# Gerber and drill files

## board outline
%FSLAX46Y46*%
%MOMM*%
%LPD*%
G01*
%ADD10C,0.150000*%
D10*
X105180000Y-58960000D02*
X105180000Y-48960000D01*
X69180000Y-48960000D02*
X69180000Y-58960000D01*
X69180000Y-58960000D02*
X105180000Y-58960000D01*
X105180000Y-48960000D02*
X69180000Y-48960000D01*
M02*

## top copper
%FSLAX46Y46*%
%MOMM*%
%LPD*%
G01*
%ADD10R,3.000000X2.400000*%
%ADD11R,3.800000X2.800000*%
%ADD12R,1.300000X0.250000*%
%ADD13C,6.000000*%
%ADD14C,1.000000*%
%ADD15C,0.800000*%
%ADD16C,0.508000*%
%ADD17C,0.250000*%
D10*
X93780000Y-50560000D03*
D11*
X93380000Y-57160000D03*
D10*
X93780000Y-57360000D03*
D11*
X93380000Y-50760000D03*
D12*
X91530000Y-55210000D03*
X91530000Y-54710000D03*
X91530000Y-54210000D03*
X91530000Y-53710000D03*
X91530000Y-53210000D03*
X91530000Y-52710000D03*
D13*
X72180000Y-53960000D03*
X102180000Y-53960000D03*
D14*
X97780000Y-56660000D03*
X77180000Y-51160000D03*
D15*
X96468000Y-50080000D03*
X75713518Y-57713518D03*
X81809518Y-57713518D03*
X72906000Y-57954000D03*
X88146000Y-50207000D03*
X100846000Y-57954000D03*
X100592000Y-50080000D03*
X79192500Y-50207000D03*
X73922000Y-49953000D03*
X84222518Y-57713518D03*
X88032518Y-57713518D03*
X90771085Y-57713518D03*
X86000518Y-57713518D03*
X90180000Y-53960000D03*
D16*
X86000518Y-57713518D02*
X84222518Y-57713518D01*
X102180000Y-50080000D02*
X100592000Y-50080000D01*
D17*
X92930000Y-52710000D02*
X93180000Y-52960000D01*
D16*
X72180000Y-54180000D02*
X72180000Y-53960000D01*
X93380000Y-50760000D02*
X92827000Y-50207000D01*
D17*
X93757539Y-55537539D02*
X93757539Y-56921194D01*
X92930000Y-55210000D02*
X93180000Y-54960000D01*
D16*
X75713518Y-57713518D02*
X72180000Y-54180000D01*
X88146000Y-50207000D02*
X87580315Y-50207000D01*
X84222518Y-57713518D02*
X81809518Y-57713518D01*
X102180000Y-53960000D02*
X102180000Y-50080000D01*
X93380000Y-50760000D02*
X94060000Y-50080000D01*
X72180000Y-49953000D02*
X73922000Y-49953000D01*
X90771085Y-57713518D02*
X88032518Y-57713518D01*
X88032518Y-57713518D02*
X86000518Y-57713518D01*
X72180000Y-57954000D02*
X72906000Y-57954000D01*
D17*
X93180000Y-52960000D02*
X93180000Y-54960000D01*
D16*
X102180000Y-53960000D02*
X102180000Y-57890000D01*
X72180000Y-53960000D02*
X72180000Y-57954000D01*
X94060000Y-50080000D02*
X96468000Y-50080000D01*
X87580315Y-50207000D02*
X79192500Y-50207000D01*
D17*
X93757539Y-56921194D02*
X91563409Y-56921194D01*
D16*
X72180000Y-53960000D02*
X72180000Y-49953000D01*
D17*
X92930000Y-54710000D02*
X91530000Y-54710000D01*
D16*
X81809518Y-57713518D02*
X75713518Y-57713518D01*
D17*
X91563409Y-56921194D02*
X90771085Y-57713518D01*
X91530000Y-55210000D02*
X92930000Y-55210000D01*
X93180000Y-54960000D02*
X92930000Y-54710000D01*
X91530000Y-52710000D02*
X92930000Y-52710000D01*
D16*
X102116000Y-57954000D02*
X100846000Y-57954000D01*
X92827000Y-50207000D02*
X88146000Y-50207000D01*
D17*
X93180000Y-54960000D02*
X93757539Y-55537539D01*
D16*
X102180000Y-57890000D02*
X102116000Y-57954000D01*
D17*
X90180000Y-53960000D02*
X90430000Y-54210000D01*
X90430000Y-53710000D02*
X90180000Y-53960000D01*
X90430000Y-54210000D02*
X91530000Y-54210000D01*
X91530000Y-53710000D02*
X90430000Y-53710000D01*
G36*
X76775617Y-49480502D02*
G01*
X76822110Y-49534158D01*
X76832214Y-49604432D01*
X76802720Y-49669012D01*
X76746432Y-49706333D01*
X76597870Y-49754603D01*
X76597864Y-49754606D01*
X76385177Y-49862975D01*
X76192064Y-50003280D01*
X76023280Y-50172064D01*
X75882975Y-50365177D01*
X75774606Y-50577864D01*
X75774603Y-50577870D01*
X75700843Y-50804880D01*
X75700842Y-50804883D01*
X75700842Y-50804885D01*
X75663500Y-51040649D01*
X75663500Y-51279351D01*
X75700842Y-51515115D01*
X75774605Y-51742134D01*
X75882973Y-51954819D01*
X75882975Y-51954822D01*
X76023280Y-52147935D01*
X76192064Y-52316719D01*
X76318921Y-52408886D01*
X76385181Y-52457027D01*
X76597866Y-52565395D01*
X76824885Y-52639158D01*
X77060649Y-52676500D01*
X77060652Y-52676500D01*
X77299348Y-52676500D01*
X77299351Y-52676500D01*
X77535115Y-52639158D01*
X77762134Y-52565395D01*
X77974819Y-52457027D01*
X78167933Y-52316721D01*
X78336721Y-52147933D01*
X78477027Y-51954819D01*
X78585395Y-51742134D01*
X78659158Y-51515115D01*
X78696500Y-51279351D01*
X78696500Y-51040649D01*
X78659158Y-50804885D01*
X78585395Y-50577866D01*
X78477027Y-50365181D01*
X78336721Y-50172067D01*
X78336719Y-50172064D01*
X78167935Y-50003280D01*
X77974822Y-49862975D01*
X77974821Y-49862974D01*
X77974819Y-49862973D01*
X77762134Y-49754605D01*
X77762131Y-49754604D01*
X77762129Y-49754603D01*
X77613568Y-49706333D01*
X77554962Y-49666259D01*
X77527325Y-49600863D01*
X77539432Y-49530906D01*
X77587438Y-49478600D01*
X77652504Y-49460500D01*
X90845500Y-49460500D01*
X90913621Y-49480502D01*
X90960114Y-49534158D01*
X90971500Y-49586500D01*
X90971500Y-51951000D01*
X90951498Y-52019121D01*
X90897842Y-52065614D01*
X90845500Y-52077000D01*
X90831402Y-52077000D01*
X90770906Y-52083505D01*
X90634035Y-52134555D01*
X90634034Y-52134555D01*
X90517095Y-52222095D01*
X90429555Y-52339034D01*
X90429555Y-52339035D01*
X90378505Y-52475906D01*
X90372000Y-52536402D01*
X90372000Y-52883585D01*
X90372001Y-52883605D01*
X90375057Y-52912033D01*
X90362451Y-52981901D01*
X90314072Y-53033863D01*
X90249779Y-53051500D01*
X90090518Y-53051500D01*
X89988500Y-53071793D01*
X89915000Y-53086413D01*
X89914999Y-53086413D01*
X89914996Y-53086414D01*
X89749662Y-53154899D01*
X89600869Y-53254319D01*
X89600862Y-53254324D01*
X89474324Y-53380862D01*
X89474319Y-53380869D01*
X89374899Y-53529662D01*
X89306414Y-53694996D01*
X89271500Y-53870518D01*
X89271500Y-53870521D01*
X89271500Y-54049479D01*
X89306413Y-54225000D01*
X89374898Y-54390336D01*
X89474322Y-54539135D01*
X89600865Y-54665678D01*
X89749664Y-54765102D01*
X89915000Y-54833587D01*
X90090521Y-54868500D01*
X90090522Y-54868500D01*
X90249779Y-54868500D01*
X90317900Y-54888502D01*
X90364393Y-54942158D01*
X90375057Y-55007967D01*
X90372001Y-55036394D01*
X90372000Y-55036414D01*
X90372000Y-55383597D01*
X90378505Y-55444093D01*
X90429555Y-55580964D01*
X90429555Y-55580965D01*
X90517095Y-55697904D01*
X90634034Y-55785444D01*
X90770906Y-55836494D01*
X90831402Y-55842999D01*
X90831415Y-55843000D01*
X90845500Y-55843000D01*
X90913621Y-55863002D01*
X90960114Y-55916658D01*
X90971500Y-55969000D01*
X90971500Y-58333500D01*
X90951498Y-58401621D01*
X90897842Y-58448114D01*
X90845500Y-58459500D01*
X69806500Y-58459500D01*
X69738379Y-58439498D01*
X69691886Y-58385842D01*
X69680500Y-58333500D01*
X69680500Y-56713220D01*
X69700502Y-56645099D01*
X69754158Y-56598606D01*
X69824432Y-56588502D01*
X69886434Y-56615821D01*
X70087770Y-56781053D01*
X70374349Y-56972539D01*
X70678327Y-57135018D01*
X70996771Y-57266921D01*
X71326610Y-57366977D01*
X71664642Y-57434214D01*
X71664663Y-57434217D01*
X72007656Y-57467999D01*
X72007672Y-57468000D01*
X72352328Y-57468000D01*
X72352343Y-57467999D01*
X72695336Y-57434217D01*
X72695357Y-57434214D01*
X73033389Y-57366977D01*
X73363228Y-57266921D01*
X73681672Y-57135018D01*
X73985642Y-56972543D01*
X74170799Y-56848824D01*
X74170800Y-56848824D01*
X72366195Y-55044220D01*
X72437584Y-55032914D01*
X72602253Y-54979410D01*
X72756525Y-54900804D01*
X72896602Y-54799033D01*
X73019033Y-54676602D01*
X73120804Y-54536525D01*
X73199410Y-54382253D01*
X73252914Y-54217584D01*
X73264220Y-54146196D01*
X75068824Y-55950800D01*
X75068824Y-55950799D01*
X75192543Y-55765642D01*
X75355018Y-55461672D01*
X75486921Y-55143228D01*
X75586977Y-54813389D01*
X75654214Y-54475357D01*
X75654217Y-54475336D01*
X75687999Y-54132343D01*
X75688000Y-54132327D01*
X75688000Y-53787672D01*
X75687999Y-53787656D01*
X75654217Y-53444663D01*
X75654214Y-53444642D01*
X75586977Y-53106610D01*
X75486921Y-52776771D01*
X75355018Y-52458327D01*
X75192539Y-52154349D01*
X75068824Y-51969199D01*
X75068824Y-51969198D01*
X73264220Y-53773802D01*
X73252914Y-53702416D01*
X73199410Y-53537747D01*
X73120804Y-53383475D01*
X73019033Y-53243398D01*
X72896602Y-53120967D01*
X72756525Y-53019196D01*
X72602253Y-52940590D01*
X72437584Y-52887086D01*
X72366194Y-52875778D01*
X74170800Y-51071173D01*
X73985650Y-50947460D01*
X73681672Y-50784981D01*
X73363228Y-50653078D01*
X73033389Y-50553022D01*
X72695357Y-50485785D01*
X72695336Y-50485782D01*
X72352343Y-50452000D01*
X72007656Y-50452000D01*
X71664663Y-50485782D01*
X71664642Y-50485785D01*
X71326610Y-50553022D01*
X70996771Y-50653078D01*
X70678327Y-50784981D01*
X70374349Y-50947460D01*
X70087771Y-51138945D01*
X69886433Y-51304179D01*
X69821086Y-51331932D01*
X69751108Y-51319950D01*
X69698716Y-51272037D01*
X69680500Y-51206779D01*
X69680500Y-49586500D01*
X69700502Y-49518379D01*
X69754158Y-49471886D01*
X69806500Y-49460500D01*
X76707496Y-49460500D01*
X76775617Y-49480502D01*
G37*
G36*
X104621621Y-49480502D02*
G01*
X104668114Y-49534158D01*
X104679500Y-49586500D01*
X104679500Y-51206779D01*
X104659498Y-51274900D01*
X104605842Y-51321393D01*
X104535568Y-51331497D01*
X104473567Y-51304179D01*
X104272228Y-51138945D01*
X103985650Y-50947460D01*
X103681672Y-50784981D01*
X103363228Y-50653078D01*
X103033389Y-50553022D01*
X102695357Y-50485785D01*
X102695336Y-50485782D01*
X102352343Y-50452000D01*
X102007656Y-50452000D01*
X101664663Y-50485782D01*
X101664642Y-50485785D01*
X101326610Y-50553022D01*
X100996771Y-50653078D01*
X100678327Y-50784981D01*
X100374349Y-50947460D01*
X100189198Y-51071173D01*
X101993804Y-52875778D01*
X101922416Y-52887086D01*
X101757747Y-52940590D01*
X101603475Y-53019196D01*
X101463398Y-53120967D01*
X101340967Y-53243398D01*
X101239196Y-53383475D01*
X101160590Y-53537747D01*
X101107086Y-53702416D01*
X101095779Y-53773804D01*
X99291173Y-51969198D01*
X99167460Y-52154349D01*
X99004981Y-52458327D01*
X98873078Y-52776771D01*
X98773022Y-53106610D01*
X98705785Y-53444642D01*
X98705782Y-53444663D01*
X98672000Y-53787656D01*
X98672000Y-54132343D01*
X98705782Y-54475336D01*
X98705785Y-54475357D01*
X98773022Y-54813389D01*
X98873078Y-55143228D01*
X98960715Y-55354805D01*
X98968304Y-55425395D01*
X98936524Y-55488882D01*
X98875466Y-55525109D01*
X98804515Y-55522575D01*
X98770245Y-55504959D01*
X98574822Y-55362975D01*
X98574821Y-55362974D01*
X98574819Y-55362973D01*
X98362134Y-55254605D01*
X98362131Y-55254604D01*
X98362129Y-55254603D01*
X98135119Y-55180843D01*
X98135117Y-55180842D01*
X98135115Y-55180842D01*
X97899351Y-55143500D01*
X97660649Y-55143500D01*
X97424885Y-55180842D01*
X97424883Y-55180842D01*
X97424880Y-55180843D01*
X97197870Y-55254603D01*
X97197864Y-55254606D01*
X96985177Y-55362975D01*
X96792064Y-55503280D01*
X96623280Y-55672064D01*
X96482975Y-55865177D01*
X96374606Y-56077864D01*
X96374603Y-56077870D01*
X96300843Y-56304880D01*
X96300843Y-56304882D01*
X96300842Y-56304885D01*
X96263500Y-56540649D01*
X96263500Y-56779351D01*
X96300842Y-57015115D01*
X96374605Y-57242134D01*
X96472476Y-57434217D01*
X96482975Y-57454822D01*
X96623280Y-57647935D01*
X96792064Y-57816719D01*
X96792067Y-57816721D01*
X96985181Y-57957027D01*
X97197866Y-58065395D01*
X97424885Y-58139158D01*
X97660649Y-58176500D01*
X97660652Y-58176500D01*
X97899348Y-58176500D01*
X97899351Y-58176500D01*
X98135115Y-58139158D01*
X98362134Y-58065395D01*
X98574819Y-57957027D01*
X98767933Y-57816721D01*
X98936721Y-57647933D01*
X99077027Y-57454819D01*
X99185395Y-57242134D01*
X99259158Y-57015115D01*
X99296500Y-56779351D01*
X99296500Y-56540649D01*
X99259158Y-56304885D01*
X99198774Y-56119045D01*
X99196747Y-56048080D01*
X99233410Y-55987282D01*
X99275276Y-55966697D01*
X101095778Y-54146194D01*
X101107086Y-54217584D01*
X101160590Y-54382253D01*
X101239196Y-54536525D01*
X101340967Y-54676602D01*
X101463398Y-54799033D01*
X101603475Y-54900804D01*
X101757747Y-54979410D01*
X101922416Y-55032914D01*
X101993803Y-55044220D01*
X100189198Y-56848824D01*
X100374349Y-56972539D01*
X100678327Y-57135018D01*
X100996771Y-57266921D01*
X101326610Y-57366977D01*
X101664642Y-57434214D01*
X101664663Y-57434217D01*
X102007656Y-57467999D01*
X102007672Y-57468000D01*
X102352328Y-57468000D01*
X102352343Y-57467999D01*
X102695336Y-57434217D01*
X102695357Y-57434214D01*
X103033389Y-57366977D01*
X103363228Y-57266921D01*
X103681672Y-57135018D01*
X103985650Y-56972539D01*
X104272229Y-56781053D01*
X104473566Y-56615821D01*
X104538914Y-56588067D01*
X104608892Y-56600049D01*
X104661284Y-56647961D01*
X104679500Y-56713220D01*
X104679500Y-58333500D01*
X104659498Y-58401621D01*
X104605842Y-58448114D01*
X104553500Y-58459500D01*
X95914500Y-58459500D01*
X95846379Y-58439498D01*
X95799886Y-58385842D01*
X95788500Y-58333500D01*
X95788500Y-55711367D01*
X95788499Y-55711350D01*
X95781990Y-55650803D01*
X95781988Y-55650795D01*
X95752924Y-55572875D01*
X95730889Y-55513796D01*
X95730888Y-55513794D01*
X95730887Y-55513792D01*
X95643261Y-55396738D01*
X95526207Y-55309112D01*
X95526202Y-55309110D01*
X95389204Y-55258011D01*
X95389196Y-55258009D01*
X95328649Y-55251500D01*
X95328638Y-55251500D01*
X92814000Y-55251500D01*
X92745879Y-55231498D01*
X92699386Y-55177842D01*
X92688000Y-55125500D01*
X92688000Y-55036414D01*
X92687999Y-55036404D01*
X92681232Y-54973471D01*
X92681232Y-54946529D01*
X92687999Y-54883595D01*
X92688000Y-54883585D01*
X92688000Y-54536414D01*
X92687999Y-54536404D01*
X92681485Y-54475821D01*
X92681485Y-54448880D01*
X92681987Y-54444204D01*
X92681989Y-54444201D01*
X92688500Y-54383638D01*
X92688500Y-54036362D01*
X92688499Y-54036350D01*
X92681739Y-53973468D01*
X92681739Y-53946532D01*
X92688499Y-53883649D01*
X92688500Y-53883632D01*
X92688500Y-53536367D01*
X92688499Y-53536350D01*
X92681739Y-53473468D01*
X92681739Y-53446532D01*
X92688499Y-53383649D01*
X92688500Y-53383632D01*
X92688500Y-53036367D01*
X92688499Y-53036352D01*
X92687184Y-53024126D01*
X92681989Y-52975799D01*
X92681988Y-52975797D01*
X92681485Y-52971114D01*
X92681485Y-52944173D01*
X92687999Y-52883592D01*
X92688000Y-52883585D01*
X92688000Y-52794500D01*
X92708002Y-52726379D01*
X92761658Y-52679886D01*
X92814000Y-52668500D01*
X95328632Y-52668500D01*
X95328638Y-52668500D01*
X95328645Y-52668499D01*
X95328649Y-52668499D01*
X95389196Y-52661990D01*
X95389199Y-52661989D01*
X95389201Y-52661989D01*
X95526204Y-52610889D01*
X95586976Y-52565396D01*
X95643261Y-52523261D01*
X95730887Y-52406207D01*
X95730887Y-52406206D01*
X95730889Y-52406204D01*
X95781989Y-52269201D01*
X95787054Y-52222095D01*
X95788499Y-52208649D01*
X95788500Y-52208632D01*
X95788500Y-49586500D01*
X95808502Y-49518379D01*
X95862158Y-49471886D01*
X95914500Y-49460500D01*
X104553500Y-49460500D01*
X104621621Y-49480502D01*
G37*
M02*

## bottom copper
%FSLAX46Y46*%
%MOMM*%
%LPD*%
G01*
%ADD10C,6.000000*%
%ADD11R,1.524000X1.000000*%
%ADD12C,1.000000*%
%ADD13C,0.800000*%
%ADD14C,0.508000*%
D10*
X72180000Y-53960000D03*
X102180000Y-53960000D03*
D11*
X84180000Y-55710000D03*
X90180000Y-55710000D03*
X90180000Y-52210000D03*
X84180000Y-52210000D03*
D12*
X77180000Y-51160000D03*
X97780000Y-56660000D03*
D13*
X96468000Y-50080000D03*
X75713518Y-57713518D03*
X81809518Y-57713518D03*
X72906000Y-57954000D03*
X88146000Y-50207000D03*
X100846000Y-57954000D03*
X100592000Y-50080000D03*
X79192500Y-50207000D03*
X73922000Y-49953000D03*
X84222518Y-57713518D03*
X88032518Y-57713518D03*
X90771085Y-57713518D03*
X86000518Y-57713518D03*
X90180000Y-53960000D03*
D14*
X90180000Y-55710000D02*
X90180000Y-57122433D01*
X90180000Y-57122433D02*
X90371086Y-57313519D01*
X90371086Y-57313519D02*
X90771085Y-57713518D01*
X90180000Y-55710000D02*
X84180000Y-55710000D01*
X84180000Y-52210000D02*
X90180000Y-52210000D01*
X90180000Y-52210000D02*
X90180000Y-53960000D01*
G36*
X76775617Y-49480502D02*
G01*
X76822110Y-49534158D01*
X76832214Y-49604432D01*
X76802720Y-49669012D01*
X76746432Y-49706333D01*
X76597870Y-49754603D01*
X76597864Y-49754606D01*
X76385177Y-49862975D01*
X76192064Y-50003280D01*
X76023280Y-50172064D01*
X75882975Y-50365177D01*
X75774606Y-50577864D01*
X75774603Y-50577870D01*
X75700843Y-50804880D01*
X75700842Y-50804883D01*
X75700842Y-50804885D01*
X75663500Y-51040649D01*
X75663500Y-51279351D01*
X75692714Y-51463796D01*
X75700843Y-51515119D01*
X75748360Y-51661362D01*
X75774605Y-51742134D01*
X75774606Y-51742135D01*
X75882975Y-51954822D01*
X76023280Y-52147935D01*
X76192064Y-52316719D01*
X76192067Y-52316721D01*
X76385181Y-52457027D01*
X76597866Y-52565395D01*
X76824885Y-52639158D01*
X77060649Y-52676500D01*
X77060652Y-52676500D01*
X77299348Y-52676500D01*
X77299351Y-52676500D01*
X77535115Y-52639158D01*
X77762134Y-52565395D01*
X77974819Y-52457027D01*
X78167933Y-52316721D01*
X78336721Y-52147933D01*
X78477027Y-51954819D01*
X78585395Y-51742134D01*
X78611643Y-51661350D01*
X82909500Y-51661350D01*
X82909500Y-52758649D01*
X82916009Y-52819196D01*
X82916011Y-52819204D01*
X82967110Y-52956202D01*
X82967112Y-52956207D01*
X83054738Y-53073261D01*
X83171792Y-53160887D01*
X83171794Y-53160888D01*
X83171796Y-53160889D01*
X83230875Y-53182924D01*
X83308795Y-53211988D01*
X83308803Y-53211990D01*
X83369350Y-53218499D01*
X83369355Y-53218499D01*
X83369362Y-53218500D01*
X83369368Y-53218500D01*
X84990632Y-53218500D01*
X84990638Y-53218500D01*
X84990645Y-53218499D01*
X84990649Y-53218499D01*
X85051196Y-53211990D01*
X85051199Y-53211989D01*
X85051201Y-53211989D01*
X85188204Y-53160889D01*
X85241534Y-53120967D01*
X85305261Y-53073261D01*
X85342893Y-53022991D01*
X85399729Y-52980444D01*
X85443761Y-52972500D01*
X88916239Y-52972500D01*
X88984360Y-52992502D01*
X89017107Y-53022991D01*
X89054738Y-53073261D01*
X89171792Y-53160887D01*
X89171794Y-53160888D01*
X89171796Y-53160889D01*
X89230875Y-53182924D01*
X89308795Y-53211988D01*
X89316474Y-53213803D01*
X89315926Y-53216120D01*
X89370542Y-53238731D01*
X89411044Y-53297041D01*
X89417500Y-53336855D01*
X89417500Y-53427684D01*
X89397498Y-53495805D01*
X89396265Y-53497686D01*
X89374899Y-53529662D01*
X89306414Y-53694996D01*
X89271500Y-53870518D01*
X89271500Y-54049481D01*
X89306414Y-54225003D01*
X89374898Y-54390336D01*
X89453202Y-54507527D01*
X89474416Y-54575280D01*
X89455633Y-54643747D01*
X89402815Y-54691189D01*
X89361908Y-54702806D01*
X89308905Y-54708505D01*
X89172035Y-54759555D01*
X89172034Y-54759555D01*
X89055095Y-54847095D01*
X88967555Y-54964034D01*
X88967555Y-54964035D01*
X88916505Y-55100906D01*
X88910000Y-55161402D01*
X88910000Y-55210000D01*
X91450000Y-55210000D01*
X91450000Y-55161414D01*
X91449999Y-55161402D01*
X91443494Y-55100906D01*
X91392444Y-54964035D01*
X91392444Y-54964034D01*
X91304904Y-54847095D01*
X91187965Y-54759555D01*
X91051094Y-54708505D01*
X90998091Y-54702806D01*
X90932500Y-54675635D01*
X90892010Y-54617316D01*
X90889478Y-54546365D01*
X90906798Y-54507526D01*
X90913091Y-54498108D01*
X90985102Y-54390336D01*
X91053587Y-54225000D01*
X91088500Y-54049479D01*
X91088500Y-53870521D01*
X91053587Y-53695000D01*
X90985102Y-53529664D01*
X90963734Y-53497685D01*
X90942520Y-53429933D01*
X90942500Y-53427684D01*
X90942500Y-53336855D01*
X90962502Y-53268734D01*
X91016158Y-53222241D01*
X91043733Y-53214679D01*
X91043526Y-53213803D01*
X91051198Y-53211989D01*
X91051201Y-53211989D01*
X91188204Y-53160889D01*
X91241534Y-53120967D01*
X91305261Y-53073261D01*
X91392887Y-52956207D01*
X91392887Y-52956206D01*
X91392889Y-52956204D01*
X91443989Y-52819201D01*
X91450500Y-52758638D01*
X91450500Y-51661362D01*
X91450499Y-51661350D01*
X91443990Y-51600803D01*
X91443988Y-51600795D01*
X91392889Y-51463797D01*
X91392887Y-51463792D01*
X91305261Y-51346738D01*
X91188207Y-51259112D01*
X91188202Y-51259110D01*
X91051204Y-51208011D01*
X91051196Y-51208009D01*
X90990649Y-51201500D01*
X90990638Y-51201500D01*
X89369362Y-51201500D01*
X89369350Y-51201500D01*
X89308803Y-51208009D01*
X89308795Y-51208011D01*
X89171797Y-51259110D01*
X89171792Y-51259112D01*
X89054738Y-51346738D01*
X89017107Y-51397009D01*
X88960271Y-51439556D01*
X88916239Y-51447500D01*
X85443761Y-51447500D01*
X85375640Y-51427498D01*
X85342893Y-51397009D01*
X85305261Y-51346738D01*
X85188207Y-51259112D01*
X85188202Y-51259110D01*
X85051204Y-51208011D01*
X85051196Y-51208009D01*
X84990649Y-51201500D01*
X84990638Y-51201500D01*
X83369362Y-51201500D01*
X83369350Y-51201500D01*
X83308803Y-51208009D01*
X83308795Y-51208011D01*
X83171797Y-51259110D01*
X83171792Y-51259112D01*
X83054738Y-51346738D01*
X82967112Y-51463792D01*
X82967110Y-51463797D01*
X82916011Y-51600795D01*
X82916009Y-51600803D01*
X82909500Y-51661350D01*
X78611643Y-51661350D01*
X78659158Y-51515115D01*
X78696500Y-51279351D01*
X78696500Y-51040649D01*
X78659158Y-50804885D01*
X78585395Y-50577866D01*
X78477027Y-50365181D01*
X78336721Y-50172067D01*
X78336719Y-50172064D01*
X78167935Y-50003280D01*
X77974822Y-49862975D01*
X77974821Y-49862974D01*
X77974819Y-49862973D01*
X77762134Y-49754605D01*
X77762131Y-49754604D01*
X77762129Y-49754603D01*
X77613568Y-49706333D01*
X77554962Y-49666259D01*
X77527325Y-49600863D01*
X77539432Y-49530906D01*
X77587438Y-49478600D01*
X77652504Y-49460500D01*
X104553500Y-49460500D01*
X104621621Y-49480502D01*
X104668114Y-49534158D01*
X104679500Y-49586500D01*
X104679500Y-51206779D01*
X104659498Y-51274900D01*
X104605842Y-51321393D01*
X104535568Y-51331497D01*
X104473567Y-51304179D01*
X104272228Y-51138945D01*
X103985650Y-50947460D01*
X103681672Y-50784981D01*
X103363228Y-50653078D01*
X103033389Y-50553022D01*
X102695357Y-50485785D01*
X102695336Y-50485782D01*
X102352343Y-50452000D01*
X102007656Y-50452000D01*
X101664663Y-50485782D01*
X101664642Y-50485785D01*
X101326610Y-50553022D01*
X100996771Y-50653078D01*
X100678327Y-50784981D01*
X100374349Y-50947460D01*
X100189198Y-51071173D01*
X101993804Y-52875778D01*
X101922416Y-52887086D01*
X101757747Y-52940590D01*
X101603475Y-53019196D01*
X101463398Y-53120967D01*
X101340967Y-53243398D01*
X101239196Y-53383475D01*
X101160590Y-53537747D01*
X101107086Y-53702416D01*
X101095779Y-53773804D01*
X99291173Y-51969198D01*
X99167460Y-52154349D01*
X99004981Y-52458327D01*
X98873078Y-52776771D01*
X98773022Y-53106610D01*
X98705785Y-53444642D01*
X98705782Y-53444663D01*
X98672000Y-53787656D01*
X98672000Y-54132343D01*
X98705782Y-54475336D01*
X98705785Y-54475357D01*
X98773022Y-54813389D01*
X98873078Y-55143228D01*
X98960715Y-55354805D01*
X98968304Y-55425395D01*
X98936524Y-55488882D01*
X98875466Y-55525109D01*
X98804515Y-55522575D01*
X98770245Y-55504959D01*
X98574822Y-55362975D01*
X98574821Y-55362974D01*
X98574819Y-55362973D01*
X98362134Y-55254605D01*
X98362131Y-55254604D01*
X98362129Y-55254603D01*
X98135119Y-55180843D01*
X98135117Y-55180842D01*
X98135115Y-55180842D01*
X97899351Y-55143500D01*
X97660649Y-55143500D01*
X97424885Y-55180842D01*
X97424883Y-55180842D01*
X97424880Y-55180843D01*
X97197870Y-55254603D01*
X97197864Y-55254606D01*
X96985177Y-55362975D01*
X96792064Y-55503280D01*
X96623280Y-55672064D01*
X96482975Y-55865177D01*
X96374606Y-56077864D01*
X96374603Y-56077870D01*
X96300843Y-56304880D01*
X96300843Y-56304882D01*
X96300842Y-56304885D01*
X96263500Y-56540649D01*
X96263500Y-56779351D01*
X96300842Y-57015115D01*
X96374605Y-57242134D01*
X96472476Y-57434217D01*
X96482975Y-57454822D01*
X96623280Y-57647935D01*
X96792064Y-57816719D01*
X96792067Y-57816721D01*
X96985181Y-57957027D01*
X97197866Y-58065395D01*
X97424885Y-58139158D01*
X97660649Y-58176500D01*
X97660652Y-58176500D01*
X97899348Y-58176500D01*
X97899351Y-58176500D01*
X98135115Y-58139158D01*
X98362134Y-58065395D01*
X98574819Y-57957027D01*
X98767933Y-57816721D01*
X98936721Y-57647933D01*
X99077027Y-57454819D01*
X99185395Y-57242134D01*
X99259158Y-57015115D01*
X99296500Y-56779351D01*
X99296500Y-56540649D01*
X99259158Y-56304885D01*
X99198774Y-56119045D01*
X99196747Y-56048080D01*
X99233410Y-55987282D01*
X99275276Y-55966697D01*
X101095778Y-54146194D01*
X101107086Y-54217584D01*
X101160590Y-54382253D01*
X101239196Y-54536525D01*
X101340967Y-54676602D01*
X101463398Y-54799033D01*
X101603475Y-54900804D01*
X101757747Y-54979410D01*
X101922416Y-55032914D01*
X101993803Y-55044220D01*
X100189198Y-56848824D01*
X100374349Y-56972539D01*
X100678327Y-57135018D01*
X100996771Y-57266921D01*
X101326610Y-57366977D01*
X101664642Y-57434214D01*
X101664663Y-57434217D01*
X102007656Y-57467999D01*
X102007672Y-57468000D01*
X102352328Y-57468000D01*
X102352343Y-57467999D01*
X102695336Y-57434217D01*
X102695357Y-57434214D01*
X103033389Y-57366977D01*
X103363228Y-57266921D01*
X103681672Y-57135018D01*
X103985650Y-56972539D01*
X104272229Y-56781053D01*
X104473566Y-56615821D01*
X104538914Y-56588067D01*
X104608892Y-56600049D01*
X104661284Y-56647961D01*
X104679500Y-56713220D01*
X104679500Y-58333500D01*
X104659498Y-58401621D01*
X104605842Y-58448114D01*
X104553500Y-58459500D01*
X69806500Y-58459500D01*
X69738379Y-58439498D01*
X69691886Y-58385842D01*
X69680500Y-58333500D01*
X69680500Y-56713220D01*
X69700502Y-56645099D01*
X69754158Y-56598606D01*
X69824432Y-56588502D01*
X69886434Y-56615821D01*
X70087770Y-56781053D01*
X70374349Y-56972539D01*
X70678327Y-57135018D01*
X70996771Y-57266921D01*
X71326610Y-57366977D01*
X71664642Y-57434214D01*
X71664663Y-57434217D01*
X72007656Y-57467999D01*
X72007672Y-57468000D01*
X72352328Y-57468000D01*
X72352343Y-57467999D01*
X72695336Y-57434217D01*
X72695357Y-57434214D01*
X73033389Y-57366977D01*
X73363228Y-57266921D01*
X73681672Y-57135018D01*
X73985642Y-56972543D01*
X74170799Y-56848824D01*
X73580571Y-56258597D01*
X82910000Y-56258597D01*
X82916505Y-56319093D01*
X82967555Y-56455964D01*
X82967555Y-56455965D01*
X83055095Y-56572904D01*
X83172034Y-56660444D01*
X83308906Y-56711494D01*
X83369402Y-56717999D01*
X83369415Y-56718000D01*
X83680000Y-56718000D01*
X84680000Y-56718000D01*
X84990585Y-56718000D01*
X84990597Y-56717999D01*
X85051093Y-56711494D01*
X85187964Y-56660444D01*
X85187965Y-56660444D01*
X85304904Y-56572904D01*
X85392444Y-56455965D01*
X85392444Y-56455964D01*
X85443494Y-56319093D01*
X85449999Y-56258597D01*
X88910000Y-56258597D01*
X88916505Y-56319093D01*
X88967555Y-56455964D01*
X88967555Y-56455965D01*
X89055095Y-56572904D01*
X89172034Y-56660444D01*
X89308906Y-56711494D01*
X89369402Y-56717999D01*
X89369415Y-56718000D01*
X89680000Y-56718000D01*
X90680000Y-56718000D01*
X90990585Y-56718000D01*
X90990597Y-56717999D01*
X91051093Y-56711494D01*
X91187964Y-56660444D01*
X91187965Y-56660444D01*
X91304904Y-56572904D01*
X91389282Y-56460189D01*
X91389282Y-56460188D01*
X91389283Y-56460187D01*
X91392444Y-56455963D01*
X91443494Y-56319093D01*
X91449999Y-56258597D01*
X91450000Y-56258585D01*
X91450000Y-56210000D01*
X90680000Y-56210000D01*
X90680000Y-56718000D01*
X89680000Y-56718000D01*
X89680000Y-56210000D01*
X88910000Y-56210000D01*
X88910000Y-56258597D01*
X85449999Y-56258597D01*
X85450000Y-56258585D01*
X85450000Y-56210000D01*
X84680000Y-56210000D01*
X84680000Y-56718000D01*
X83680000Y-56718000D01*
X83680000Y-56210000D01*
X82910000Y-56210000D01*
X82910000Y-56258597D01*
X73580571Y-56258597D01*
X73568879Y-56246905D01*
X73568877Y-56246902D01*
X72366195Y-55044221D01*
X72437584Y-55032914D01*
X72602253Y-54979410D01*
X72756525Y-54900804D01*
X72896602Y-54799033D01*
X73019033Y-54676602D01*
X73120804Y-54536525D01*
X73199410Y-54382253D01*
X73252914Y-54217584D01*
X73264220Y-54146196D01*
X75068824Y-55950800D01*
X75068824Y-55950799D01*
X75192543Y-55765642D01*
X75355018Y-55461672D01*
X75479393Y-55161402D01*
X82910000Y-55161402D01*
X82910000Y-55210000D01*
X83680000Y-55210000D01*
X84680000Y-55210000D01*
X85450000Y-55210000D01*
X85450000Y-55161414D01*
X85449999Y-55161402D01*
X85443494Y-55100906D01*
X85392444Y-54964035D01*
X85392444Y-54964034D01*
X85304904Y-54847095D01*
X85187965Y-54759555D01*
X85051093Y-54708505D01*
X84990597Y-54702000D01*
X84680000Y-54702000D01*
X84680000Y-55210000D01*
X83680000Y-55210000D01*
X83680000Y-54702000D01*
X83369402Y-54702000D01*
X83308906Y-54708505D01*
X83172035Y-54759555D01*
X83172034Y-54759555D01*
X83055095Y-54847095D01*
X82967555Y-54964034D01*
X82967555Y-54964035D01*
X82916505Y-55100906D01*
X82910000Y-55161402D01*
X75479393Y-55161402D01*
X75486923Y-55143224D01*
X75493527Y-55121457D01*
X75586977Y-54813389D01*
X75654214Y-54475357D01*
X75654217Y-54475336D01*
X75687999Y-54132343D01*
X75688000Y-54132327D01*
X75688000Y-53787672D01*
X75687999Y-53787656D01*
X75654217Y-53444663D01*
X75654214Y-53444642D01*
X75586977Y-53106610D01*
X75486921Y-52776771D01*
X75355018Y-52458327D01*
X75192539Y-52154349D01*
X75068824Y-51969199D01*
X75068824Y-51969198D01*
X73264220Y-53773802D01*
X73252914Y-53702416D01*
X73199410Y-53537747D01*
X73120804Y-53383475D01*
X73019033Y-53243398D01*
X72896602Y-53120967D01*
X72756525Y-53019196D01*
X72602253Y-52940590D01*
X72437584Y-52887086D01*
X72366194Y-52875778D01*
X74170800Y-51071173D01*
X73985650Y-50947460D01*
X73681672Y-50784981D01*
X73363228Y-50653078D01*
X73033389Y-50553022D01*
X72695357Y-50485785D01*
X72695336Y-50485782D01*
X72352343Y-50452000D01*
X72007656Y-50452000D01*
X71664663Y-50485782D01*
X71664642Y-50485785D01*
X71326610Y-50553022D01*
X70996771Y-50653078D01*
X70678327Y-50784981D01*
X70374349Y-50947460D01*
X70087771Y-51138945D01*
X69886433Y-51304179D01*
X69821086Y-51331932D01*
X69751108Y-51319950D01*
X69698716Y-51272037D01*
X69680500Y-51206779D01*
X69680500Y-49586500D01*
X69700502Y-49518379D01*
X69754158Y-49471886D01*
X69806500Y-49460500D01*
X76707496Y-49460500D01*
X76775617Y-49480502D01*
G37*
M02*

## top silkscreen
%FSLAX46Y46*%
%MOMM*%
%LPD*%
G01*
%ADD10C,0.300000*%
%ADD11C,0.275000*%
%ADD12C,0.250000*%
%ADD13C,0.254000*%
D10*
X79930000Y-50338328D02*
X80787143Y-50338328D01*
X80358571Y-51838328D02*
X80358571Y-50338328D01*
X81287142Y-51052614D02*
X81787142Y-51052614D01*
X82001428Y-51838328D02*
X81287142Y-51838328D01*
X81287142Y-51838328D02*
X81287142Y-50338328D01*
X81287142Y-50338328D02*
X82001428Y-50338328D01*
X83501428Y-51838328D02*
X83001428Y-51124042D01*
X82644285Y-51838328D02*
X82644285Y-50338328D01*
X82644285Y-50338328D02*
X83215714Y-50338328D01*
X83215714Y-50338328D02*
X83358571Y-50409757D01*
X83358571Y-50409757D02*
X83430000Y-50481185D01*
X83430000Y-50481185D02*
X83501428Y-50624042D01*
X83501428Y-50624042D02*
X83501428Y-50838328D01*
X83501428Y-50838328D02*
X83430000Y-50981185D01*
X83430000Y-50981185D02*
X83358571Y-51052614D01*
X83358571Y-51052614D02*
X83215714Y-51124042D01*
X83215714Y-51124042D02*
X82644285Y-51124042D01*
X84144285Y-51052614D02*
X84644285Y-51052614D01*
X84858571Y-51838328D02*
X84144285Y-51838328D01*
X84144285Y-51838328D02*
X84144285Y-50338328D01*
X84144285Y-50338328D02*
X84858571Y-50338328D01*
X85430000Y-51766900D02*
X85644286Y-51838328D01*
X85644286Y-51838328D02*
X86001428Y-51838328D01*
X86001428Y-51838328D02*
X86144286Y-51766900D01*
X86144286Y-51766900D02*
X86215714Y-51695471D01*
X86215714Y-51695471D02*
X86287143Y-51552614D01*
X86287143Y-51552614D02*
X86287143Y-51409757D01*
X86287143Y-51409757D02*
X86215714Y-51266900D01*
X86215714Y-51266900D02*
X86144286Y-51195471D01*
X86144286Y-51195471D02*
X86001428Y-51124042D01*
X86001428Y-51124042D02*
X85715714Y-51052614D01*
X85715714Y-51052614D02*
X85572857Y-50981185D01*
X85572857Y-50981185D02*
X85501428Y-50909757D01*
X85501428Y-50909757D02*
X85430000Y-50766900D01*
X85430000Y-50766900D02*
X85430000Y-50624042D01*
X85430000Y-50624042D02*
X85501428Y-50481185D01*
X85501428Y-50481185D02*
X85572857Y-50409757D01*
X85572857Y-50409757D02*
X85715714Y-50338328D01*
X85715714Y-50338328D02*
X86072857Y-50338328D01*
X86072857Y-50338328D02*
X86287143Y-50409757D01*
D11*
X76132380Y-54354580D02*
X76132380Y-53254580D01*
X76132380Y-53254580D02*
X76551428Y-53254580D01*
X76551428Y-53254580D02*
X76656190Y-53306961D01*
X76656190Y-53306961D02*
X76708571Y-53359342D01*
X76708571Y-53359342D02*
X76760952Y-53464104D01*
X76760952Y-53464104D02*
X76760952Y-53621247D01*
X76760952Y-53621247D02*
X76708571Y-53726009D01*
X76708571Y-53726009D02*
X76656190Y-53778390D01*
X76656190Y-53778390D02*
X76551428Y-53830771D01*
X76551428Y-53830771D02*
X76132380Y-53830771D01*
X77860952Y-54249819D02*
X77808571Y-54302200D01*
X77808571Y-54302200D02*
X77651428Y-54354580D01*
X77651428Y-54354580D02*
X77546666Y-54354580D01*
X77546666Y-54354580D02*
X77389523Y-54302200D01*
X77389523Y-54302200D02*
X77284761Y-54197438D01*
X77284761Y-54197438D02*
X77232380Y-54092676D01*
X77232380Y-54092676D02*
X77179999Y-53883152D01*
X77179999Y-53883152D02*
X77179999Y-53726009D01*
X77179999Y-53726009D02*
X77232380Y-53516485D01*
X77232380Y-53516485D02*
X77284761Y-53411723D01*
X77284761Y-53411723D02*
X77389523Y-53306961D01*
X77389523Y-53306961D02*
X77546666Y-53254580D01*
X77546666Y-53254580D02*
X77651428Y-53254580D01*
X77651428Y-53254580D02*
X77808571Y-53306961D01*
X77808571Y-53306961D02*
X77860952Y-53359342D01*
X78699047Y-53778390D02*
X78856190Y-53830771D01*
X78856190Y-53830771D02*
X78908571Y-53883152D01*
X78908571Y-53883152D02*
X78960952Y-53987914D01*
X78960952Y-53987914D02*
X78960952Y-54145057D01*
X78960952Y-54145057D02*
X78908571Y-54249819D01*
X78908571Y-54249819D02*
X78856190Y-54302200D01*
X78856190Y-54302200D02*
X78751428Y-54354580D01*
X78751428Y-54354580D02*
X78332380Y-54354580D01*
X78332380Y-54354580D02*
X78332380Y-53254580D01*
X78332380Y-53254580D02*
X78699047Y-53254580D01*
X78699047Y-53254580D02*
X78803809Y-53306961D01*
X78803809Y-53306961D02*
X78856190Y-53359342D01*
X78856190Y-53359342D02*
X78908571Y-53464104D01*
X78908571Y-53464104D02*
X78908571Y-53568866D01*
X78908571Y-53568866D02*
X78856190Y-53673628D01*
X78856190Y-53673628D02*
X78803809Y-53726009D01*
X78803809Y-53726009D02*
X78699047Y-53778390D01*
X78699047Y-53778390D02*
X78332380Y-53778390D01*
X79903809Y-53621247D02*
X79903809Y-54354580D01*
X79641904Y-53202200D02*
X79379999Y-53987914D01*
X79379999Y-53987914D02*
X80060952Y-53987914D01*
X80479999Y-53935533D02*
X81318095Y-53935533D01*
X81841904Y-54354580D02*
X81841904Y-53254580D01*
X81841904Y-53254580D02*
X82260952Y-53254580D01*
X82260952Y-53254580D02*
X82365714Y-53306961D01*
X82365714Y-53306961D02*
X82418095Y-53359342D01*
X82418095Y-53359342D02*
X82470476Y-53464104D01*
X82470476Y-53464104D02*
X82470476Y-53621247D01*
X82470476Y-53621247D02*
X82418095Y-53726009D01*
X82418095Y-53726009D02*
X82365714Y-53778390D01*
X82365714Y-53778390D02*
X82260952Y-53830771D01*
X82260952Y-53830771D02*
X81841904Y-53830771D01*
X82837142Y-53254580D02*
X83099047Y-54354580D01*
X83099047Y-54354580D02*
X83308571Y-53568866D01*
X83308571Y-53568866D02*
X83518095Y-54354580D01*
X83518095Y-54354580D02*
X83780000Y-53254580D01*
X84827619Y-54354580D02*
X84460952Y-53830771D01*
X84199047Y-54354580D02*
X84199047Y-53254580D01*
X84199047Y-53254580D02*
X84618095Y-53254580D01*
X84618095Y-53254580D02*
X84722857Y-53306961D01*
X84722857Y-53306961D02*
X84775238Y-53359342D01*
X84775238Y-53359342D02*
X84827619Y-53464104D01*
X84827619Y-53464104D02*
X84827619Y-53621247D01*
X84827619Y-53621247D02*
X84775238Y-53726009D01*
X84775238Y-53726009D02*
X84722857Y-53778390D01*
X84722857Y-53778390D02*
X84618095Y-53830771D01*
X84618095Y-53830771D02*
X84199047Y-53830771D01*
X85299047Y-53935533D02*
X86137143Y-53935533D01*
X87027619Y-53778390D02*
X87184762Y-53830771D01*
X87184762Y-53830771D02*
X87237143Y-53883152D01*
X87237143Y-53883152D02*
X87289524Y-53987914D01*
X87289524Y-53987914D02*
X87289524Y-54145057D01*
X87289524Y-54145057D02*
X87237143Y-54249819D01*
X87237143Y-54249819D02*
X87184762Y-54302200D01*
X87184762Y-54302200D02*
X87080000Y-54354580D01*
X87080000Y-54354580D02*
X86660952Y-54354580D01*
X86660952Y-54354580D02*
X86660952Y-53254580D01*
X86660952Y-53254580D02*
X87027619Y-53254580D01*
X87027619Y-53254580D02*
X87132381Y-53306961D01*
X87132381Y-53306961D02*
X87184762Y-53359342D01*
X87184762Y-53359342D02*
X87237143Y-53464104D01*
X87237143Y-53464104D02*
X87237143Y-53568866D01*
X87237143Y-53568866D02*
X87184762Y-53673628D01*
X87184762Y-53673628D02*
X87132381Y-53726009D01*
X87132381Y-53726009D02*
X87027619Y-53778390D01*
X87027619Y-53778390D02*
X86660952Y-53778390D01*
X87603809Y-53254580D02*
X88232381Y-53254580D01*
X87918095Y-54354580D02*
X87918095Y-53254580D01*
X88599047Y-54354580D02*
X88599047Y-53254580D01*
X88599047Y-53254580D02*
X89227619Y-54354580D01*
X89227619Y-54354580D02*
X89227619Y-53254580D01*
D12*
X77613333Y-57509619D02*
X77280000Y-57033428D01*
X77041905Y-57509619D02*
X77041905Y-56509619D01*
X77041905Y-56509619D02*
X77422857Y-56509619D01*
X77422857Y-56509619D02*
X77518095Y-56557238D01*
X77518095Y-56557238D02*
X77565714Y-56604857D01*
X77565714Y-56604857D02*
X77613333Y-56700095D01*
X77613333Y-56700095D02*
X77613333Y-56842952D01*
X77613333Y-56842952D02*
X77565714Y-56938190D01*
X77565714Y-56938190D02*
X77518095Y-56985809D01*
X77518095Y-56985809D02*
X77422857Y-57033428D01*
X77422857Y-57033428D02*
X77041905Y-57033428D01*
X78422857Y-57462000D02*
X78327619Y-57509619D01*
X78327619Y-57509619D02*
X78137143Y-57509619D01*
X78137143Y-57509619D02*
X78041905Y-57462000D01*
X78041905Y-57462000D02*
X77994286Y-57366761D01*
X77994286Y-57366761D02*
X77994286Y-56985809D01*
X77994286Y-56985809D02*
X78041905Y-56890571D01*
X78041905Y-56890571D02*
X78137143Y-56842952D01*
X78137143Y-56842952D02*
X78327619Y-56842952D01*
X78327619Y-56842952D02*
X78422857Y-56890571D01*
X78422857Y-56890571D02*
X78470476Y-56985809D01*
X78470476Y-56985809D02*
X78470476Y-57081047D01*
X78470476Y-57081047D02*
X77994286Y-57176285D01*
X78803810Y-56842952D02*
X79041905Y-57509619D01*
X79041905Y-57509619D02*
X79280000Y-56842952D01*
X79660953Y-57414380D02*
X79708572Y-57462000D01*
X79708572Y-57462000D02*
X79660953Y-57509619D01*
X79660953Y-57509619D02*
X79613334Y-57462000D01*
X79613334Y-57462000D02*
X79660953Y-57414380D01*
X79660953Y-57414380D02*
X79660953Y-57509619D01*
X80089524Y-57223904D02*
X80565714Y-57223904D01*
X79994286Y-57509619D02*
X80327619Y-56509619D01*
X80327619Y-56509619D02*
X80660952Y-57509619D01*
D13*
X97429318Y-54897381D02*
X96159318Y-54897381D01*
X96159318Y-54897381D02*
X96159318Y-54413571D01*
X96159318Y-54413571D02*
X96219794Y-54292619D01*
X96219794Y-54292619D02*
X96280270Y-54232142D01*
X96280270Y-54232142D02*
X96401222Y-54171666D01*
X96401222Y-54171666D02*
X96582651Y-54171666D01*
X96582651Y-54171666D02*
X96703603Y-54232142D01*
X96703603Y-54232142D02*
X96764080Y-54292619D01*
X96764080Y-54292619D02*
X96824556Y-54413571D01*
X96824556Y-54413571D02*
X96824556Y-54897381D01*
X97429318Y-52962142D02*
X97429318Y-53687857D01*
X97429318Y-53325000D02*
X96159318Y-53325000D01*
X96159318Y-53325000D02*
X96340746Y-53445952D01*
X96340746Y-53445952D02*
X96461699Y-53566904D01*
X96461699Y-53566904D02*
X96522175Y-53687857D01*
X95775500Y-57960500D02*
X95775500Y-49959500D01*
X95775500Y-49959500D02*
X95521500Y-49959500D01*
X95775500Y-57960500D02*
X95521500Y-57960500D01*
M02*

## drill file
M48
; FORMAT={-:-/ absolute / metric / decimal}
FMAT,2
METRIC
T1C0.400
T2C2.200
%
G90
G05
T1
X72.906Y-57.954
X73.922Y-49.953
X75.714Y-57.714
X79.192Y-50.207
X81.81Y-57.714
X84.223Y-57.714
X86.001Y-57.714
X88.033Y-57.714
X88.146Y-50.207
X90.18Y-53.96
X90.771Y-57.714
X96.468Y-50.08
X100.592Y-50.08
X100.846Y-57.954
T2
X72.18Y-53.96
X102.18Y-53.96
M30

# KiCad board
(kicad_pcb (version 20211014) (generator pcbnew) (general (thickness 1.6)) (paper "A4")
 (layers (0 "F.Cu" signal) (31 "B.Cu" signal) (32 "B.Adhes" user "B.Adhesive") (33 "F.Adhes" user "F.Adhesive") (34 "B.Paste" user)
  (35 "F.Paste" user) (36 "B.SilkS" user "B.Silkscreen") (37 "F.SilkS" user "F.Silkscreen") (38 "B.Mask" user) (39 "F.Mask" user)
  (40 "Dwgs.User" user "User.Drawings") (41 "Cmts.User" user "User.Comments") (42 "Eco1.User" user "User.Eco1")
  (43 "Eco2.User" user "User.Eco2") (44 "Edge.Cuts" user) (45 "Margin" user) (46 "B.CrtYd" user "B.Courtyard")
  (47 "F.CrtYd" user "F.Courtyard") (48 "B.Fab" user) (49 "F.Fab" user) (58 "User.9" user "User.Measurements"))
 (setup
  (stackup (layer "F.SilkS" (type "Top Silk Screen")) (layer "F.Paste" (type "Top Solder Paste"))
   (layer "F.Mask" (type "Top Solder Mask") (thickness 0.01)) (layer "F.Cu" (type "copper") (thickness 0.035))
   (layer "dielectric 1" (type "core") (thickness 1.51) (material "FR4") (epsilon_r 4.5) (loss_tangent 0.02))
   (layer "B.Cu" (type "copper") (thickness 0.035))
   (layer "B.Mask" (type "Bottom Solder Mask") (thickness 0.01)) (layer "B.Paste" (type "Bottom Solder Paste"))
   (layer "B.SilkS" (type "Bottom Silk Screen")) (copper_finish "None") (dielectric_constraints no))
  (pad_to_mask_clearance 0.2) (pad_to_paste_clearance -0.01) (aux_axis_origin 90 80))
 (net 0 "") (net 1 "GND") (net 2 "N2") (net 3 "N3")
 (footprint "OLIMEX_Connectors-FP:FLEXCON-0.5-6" (layer "F.Cu") (at 93.68 53.96 90)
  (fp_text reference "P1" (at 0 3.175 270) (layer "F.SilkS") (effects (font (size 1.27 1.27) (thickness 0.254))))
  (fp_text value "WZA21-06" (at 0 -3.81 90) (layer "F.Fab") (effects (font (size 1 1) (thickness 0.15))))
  (fp_line (start -4.0005 2.0955) (end 4.0005 2.0955) (layer "F.SilkS") (width 0.254))
  (fp_line (start 4.0005 2.0955) (end 4.0005 1.8415) (layer "F.SilkS") (width 0.254))
  (fp_line (start -4.0005 2.0955) (end -4.0005 1.8415) (layer "F.SilkS") (width 0.254))
  (pad "0" smd rect locked (at 3.4 0.1 90) (size 2.4 3) (layers "F.Cu" "F.Paste" "F.Mask") (solder_mask_margin -0.01)
   (solder_paste_margin -0.01))
  (pad "0" smd rect locked (at -3.2 -0.3 90) (size 2.8 3.8) (layers "F.Cu") (solder_mask_margin -0.1) (solder_paste_margin -0.1))
  (pad "0" smd rect locked (at -3.4 0.1 90) (size 2.4 3) (layers "F.Cu" "F.Paste" "F.Mask") (solder_mask_margin -0.01)
   (solder_paste_margin -0.01))
  (pad "0" smd rect locked (at 3.2 -0.3 90) (size 2.8 3.8) (layers "F.Cu") (solder_mask_margin -0.1) (solder_paste_margin -0.1))
  (pad "1" smd rect locked (at -1.25 -2.15 90) (size 0.25 1.3) (layers "F.Cu" "F.Paste" "F.Mask") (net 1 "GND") (solder_mask_margin 0.0508)
   (solder_paste_margin -0.01))
  (pad "2" smd rect locked (at -0.75 -2.15 90) (size 0.25 1.3) (layers "F.Cu" "F.Paste" "F.Mask") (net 1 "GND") (solder_mask_margin 0.0508)
   (solder_paste_margin -0.01))
  (pad "3" smd rect locked (at -0.25 -2.15 90) (size 0.25 1.3) (layers "F.Cu" "F.Paste" "F.Mask") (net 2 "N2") (solder_mask_margin 0.0508)
   (solder_paste_margin -0.01))
  (pad "4" smd rect locked (at 0.25 -2.15 90) (size 0.25 1.3) (layers "F.Cu" "F.Paste" "F.Mask") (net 2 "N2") (solder_mask_margin 0.0508)
   (solder_paste_margin -0.01))
  (pad "5" smd rect locked (at 0.75 -2.15 90) (size 0.25 1.3) (layers "F.Cu" "F.Paste" "F.Mask") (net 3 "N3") (solder_mask_margin 0.0508)
   (solder_paste_margin -0.01))
  (pad "6" smd rect locked (at 1.25 -2.15 90) (size 0.25 1.3) (layers "F.Cu" "F.Paste" "F.Mask") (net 1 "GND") (solder_mask_margin 0.0508)
   (solder_paste_margin -0.01)))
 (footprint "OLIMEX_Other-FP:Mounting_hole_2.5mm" (layer "F.Cu") (at 72.18 53.96)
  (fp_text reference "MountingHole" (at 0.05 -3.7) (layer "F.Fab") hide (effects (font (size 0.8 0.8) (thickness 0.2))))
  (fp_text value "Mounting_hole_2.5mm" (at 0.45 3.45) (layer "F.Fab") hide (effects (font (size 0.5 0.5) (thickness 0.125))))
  (pad "" thru_hole circle locked (at 0 0) (size 6 6) (drill 2.2) (layers *.Cu *.Mask) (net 1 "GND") (clearance 1.55)))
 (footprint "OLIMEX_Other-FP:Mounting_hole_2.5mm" (layer "F.Cu") (at 102.18 53.96)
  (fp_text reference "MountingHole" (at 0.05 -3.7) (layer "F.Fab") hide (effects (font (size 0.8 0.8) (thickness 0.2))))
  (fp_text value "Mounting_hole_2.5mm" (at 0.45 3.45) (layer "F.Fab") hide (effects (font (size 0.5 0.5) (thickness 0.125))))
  (pad "" thru_hole circle locked (at 0 0) (size 6 6) (drill 2.2) (layers *.Cu *.Mask) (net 1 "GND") (clearance 1.55)))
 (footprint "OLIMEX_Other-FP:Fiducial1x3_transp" (layer "F.Cu") (at 97.78 56.66)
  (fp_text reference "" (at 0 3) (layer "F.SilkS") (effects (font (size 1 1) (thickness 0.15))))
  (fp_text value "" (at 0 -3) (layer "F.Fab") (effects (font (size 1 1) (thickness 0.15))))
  (pad "Fid1" connect circle locked (at 0 0) (size 1 1) (layers "F.Cu" "F.Mask") (solder_mask_margin 0.127) (clearance 1.016)
   (zone_connect 0)))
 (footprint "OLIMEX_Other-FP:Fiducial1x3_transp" (layer "F.Cu") (at 77.18 51.16)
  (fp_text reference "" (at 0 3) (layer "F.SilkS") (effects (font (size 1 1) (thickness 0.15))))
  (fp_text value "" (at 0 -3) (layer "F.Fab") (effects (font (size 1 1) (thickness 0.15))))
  (pad "Fid1" connect circle locked (at 0 0) (size 1 1) (layers "F.Cu" "F.Mask") (solder_mask_margin 0.127) (clearance 1.016)
   (zone_connect 0)))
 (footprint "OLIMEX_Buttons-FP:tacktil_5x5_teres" (layer "B.Cu") (at 87.18 53.96)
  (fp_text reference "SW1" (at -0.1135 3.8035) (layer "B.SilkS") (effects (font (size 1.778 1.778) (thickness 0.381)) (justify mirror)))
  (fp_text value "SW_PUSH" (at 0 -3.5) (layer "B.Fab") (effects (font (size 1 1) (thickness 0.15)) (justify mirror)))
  (pad "1" smd rect locked (at -3 1.75) (size 1.524 1) (layers "B.Cu" "B.Paste" "B.Mask") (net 1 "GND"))
  (pad "1" smd rect locked (at 3 1.75) (size 1.524 1) (layers "B.Cu" "B.Paste" "B.Mask") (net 1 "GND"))
  (pad "2" smd rect locked (at 3 -1.75) (size 1.524 1) (layers "B.Cu" "B.Paste" "B.Mask") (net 2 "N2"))
  (pad "2" smd rect locked (at -3 -1.75) (size 1.524 1) (layers "B.Cu" "B.Paste" "B.Mask") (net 2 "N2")))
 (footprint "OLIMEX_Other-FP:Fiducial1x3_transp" (layer "B.Cu") (at 77.18 51.16)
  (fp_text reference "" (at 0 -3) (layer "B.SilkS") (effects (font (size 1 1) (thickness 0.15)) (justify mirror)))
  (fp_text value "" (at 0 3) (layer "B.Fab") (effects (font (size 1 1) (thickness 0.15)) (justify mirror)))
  (pad "Fid1" connect circle locked (at 0 0) (size 1 1) (layers "B.Cu" "B.Mask") (solder_mask_margin 0.127) (clearance 1.016)
   (zone_connect 0)))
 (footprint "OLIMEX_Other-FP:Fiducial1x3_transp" (layer "B.Cu") (at 97.78 56.66)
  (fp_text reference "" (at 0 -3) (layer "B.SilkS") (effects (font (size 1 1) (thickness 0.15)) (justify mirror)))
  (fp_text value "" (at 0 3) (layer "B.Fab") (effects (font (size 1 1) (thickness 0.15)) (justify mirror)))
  (pad "Fid1" connect circle locked (at 0 0) (size 1 1) (layers "B.Cu" "B.Mask") (solder_mask_margin 0.127) (clearance 1.016)
   (zone_connect 0)))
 (gr_line (start 105.18 58.96) (end 105.18 48.96) (layer "Edge.Cuts") (width 0.15))
 (gr_line (start 69.18 48.96) (end 69.18 58.96) (layer "Edge.Cuts") (width 0.15))
 (gr_line (start 69.18 58.96) (end 105.18 58.96) (layer "Edge.Cuts") (width 0.15))
 (gr_line (start 105.18 48.96) (end 69.18 48.96) (layer "Edge.Cuts") (width 0.15))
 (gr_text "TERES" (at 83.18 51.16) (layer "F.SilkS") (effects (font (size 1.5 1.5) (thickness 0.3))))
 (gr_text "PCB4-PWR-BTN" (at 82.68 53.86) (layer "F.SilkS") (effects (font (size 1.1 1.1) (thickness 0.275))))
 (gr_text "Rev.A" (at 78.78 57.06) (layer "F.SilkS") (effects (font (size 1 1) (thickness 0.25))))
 (segment (start 86.000518 57.713518) (end 84.222518 57.713518) (width 0.508) (layer "F.Cu") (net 1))
 (segment (start 102.18 50.08) (end 100.592 50.08) (width 0.508) (layer "F.Cu") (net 1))
 (segment (start 92.93 52.71) (end 93.18 52.96) (width 0.25) (layer "F.Cu") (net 1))
 (segment (start 72.18 54.18) (end 72.18 53.96) (width 0.508) (layer "F.Cu") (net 1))
 (segment (start 93.38 50.76) (end 92.827 50.207) (width 0.508) (layer "F.Cu") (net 1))
 (segment (start 93.757539 55.537539) (end 93.757539 56.921194) (width 0.25) (layer "F.Cu") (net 1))
 (segment (start 92.93 55.21) (end 93.18 54.96) (width 0.25) (layer "F.Cu") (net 1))
 (segment (start 75.713518 57.713518) (end 72.18 54.18) (width 0.508) (layer "F.Cu") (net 1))
 (segment (start 88.146 50.207) (end 87.580315 50.207) (width 0.508) (layer "F.Cu") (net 1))
 (segment (start 84.222518 57.713518) (end 81.809518 57.713518) (width 0.508) (layer "F.Cu") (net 1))
 (segment (start 102.18 53.96) (end 102.18 50.08) (width 0.508) (layer "F.Cu") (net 1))
 (segment (start 93.38 50.76) (end 94.06 50.08) (width 0.508) (layer "F.Cu") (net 1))
 (segment (start 72.18 49.953) (end 73.922 49.953) (width 0.508) (layer "F.Cu") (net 1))
 (segment (start 90.771085 57.713518) (end 88.032518 57.713518) (width 0.508) (layer "F.Cu") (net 1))
 (segment (start 88.032518 57.713518) (end 86.000518 57.713518) (width 0.508) (layer "F.Cu") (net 1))
 (segment (start 72.18 57.954) (end 72.906 57.954) (width 0.508) (layer "F.Cu") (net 1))
 (segment (start 93.18 52.96) (end 93.18 54.96) (width 0.25) (layer "F.Cu") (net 1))
 (segment (start 102.18 53.96) (end 102.18 57.89) (width 0.508) (layer "F.Cu") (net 1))
 (segment (start 72.18 53.96) (end 72.18 57.954) (width 0.508) (layer "F.Cu") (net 1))
 (segment (start 94.06 50.08) (end 96.468 50.08) (width 0.508) (layer "F.Cu") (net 1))
 (segment (start 87.580315 50.207) (end 79.1925 50.207) (width 0.508) (layer "F.Cu") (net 1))
 (segment (start 93.757539 56.921194) (end 91.563409 56.921194) (width 0.25) (layer "F.Cu") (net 1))
 (segment (start 72.18 53.96) (end 72.18 49.953) (width 0.508) (layer "F.Cu") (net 1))
 (segment (start 92.93 54.71) (end 91.53 54.71) (width 0.25) (layer "F.Cu") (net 1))
 (segment (start 81.809518 57.713518) (end 75.713518 57.713518) (width 0.508) (layer "F.Cu") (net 1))
 (segment (start 91.563409 56.921194) (end 90.771085 57.713518) (width 0.25) (layer "F.Cu") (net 1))
 (segment (start 91.53 55.21) (end 92.93 55.21) (width 0.25) (layer "F.Cu") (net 1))
 (segment (start 93.18 54.96) (end 92.93 54.71) (width 0.25) (layer "F.Cu") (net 1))
 (segment (start 91.53 52.71) (end 92.93 52.71) (width 0.25) (layer "F.Cu") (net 1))
 (segment (start 102.116 57.954) (end 100.846 57.954) (width 0.508) (layer "F.Cu") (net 1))
 (segment (start 92.827 50.207) (end 88.146 50.207) (width 0.508) (layer "F.Cu") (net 1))
 (segment (start 93.18 54.96) (end 93.757539 55.537539) (width 0.25) (layer "F.Cu") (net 1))
 (segment (start 102.18 57.89) (end 102.116 57.954) (width 0.508) (layer "F.Cu") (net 1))
 (via (at 96.468 50.08) (size 0.8) (drill 0.4) (layers "F.Cu" "B.Cu") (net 1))
 (via (at 75.713518 57.713518) (size 0.8) (drill 0.4) (layers "F.Cu" "B.Cu") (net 1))
 (via (at 81.809518 57.713518) (size 0.8) (drill 0.4) (layers "F.Cu" "B.Cu") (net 1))
 (via (at 72.906 57.954) (size 0.8) (drill 0.4) (layers "F.Cu" "B.Cu") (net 1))
 (via (at 88.146 50.207) (size 0.8) (drill 0.4) (layers "F.Cu" "B.Cu") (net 1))
 (via (at 100.846 57.954) (size 0.8) (drill 0.4) (layers "F.Cu" "B.Cu") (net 1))
 (via (at 100.592 50.08) (size 0.8) (drill 0.4) (layers "F.Cu" "B.Cu") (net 1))
 (via (at 79.1925 50.207) (size 0.8) (drill 0.4) (layers "F.Cu" "B.Cu") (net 1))
 (via (at 73.922 49.953) (size 0.8) (drill 0.4) (layers "F.Cu" "B.Cu") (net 1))
 (via (at 84.222518 57.713518) (size 0.8) (drill 0.4) (layers "F.Cu" "B.Cu") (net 1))
 (via (at 88.032518 57.713518) (size 0.8) (drill 0.4) (layers "F.Cu" "B.Cu") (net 1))
 (via (at 90.771085 57.713518) (size 0.8) (drill 0.4) (layers "F.Cu" "B.Cu") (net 1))
 (via (at 86.000518 57.713518) (size 0.8) (drill 0.4) (layers "F.Cu" "B.Cu") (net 1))
 (segment (start 90.18 55.71) (end 90.18 57.122433) (width 0.508) (layer "B.Cu") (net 1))
 (segment (start 90.18 57.122433) (end 90.371086 57.313519) (width 0.508) (layer "B.Cu") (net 1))
 (segment (start 90.371086 57.313519) (end 90.771085 57.713518) (width 0.508) (layer "B.Cu") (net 1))
 (segment (start 90.18 55.71) (end 84.18 55.71) (width 0.508) (layer "B.Cu") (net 1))
 (segment (start 90.18 53.96) (end 90.43 54.21) (width 0.25) (layer "F.Cu") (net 2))
 (segment (start 90.43 53.71) (end 90.18 53.96) (width 0.25) (layer "F.Cu") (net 2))
 (segment (start 90.43 54.21) (end 91.53 54.21) (width 0.25) (layer "F.Cu") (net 2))
 (segment (start 91.53 53.71) (end 90.43 53.71) (width 0.25) (layer "F.Cu") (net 2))
 (via (at 90.18 53.96) (size 0.8) (drill 0.4) (layers "F.Cu" "B.Cu") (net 2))
 (segment (start 84.18 52.21) (end 90.18 52.21) (width 0.508) (layer "B.Cu") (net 2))
 (segment (start 90.18 52.21) (end 90.18 53.96) (width 0.508) (layer "B.Cu") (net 2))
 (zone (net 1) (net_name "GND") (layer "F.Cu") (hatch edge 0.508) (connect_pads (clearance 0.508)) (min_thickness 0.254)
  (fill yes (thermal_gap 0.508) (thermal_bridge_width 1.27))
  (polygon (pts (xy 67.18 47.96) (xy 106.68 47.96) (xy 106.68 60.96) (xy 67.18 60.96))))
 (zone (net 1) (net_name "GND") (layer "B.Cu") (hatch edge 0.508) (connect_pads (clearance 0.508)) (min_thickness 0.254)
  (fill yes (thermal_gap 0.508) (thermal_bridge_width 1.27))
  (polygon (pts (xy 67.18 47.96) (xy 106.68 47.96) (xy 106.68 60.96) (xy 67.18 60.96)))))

